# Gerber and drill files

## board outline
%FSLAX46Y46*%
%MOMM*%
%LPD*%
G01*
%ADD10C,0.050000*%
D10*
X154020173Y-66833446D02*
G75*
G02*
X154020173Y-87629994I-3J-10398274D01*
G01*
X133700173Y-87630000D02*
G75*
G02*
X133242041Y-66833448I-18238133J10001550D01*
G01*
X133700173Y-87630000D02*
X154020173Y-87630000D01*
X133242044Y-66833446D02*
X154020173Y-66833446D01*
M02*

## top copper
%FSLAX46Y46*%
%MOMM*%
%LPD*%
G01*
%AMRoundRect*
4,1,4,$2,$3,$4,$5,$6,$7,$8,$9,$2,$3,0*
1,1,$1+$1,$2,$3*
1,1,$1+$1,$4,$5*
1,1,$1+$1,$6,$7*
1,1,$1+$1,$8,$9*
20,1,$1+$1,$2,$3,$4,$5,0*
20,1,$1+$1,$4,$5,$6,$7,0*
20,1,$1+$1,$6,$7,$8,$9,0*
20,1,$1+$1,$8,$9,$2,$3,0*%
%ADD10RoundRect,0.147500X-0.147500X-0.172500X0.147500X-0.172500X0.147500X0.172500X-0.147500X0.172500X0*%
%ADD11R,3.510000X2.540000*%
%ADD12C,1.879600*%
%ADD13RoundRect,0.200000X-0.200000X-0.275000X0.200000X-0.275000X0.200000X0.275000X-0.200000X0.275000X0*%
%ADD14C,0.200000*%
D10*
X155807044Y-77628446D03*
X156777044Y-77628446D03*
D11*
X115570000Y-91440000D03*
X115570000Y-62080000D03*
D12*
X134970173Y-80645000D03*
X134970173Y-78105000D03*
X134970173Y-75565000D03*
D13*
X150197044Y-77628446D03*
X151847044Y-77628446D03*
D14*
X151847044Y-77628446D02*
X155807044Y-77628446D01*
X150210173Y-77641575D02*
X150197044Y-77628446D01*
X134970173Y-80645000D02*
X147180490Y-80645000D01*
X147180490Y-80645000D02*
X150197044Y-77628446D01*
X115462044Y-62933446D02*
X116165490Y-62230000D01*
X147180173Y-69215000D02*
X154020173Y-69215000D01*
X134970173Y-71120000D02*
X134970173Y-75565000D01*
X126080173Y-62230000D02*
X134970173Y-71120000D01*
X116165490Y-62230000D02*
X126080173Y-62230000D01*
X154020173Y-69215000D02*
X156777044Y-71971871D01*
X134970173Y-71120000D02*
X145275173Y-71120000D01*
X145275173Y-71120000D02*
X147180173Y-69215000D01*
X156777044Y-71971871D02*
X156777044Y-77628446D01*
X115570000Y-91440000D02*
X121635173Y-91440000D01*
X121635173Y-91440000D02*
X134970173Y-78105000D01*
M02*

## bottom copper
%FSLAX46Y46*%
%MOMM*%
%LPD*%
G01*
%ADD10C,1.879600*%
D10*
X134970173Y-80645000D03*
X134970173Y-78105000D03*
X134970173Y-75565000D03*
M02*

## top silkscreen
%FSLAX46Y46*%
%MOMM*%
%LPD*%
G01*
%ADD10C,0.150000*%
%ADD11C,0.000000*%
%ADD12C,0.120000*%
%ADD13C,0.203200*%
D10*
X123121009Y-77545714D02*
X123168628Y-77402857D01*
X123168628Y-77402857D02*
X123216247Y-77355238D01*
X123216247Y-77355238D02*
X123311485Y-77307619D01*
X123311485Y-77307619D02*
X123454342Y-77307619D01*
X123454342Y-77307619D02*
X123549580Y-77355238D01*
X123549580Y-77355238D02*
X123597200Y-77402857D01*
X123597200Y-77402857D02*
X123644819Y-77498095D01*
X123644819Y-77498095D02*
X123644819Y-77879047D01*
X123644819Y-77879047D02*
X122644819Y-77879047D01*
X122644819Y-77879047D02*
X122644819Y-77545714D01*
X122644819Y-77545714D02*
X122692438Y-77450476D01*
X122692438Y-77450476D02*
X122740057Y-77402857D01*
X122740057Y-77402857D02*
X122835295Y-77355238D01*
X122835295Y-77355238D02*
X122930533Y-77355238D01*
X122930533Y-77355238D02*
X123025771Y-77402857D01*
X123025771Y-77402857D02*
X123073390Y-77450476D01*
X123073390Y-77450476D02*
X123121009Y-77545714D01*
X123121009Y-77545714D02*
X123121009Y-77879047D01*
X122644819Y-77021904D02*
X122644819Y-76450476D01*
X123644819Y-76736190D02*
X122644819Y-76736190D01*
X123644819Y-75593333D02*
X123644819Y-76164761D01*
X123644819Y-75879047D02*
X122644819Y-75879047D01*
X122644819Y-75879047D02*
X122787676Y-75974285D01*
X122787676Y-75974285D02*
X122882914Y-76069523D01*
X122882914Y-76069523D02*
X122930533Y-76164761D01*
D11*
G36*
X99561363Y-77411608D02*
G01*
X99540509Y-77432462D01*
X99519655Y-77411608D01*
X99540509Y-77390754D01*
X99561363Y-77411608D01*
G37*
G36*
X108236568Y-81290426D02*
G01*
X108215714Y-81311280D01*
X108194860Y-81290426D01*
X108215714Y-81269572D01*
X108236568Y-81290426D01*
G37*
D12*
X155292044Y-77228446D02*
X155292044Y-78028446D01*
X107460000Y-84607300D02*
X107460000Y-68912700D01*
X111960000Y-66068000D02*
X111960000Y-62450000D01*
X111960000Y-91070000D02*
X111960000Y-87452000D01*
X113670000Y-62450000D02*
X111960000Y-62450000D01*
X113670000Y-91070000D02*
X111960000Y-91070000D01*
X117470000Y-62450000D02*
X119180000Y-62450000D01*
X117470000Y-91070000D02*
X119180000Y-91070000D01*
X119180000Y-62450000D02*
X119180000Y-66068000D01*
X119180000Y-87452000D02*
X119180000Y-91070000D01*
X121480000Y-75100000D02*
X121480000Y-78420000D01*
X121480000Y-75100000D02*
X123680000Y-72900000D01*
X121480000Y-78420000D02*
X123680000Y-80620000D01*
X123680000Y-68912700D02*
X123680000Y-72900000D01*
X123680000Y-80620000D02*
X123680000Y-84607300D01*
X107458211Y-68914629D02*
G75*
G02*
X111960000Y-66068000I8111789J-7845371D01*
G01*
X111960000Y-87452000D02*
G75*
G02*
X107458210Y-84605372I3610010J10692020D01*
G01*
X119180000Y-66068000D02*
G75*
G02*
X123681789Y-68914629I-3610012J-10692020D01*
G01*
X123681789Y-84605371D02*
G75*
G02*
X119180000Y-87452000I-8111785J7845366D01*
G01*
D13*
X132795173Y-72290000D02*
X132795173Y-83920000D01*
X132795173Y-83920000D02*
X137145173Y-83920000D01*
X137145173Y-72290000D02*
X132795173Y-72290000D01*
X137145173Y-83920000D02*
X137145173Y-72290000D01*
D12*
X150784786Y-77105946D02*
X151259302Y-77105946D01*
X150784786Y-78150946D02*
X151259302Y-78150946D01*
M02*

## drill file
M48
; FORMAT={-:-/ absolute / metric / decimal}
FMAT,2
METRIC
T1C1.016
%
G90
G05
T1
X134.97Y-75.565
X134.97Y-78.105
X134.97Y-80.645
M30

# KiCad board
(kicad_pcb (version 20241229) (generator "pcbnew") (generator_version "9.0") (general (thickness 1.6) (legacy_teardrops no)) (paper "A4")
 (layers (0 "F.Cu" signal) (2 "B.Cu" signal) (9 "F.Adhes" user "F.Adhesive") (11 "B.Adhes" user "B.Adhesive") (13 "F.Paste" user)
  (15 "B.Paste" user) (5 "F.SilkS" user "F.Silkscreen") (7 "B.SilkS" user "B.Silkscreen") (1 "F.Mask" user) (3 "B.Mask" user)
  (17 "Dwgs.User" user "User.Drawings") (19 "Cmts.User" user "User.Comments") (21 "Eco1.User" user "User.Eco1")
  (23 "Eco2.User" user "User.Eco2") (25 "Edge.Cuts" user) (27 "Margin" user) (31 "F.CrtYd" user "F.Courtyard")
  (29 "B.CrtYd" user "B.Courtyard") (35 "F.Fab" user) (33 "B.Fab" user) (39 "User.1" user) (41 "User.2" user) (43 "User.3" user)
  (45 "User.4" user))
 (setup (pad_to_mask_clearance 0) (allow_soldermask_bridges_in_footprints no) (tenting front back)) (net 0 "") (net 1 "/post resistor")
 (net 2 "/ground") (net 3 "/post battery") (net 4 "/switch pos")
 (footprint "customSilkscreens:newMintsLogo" (layer "F.Cu") (at 115.285173 74.93)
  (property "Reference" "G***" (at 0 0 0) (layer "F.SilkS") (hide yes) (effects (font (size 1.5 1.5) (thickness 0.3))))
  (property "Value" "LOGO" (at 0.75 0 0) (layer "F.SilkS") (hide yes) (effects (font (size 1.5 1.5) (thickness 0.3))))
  (fp_poly
   (pts (xy -15.72381 2.481608) (xy -15.744664 2.502462) (xy -15.765518 2.481608) (xy -15.744664 2.460754)) (stroke (width 0) (type solid))
   (fill yes) (layer "F.SilkS"))
  (fp_poly
   (pts (xy -7.048605 6.360426) (xy -7.069459 6.38128) (xy -7.090313 6.360426) (xy -7.069459 6.339572)) (stroke (width 0) (type solid))
   (fill yes) (layer "F.SilkS")))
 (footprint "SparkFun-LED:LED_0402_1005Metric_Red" (layer "F.Cu") (at 156.292044 77.628446)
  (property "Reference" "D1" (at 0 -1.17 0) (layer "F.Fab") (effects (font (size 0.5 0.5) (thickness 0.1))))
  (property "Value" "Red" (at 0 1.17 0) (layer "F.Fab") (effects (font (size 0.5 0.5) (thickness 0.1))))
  (fp_line (start -1 -0.4) (end -1 0.4) (stroke (width 0.12) (type solid)) (layer "F.SilkS"))
  (pad "1" smd roundrect (at -0.485 0) (size 0.59 0.64) (layers "F.Cu" "F.Mask" "F.Paste") (roundrect_rratio 0.25) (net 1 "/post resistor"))
  (pad "2" smd roundrect (at 0.485 0) (size 0.59 0.64) (layers "F.Cu" "F.Mask" "F.Paste") (roundrect_rratio 0.25) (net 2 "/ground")))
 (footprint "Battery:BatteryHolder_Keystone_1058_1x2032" (layer "F.Cu") (at 115.57 76.76 90)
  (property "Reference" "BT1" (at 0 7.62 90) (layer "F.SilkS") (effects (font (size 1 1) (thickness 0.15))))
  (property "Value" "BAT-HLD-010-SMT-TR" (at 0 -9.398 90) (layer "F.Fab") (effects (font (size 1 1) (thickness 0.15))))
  (fp_line (start -7.8473 -8.11) (end 7.8473 -8.11) (stroke (width 0.12) (type solid)) (layer "F.SilkS"))
  (fp_line (start 10.692 -3.61) (end 14.31 -3.61) (stroke (width 0.12) (type solid)) (layer "F.SilkS"))
  (fp_line (start -14.31 -3.61) (end -10.692 -3.61) (stroke (width 0.12) (type solid)) (layer "F.SilkS"))
  (fp_line (start 14.31 -1.9) (end 14.31 -3.61) (stroke (width 0.12) (type solid)) (layer "F.SilkS"))
  (fp_line (start -14.31 -1.9) (end -14.31 -3.61) (stroke (width 0.12) (type solid)) (layer "F.SilkS"))
  (fp_line (start 14.31 1.9) (end 14.31 3.61) (stroke (width 0.12) (type solid)) (layer "F.SilkS"))
  (fp_line (start -14.31 1.9) (end -14.31 3.61) (stroke (width 0.12) (type solid)) (layer "F.SilkS"))
  (fp_line (start 14.31 3.61) (end 10.692 3.61) (stroke (width 0.12) (type solid)) (layer "F.SilkS"))
  (fp_line (start -10.692 3.61) (end -14.31 3.61) (stroke (width 0.12) (type solid)) (layer "F.SilkS"))
  (fp_line (start 1.66 5.91) (end -1.66 5.91) (stroke (width 0.12) (type solid)) (layer "F.SilkS"))
  (fp_line (start 1.66 5.91) (end 3.86 8.11) (stroke (width 0.12) (type solid)) (layer "F.SilkS"))
  (fp_line (start -1.66 5.91) (end -3.86 8.11) (stroke (width 0.12) (type solid)) (layer "F.SilkS"))
  (fp_line (start 7.8473 8.11) (end 3.86 8.11) (stroke (width 0.12) (type solid)) (layer "F.SilkS"))
  (fp_line (start -3.86 8.11) (end -7.8473 8.11) (stroke (width 0.12) (type solid)) (layer "F.SilkS"))
  (fp_arc (start 7.845371 -8.111789) (mid 9.538085 -6.031244) (end 10.692 -3.61) (stroke (width 0.12) (type solid)) (layer "F.SilkS"))
  (fp_arc (start -10.692 -3.61) (mid -9.538084 -6.031244) (end -7.845371 -8.111789) (stroke (width 0.12) (type solid)) (layer "F.SilkS"))
  (fp_arc (start 10.692 3.61) (mid 9.538084 6.031244) (end 7.845371 8.111789) (stroke (width 0.12) (type solid)) (layer "F.SilkS"))
  (fp_arc (start -7.845371 8.111789) (mid -9.538085 6.031244) (end -10.692 3.61) (stroke (width 0.12) (type solid)) (layer "F.SilkS"))
  (pad "1" smd rect (at -14.68 0 90) (size 2.54 3.51) (layers "F.Cu" "F.Mask" "F.Paste") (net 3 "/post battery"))
  (pad "2" smd rect (at 14.68 0 90) (size 2.54 3.51) (layers "F.Cu" "F.Mask" "F.Paste") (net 2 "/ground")))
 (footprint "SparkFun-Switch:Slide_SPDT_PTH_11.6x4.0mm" (layer "F.Cu") (at 134.970173 78.105 180)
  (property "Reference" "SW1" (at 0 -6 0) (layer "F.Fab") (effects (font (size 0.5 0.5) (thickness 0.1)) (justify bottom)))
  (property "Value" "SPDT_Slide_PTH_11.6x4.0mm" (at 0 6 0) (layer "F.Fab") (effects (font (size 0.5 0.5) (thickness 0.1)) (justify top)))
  (fp_line (start 2.175 5.815) (end 2.175 -5.815) (stroke (width 0.2032) (type solid)) (layer "F.SilkS"))
  (fp_line (start 2.175 -5.815) (end -2.175 -5.815) (stroke (width 0.2032) (type solid)) (layer "F.SilkS"))
  (fp_line (start -2.175 5.815) (end 2.175 5.815) (stroke (width 0.2032) (type solid)) (layer "F.SilkS"))
  (fp_line (start -2.175 -5.815) (end -2.175 5.815) (stroke (width 0.2032) (type solid)) (layer "F.SilkS"))
  (pad "1" thru_hole circle (at 0 -2.54 180) (size 1.8796 1.8796) (drill 1.016) (layers "*.Cu" "*.Mask") (remove_unused_layers no)
   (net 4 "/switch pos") (thermal_bridge_angle 0))
  (pad "2" thru_hole circle (at 0 0 180) (size 1.8796 1.8796) (drill 1.016) (layers "*.Cu" "*.Mask") (remove_unused_layers no)
   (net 3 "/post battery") (thermal_bridge_angle 0))
  (pad "3" thru_hole circle (at 0 2.54 180) (size 1.8796 1.8796) (drill 1.016) (layers "*.Cu" "*.Mask") (remove_unused_layers no)
   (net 2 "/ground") (thermal_bridge_angle 0)))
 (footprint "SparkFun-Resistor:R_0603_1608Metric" (layer "F.Cu") (at 151.022044 77.628446)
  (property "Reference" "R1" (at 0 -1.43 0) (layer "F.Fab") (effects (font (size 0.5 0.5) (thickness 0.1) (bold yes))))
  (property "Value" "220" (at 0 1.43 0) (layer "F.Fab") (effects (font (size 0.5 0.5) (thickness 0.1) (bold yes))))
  (fp_line (start -0.237258 -0.5225) (end 0.237258 -0.5225) (stroke (width 0.12) (type solid)) (layer "F.SilkS"))
  (fp_line (start -0.237258 0.5225) (end 0.237258 0.5225) (stroke (width 0.12) (type solid)) (layer "F.SilkS"))
  (pad "1" smd roundrect (at -0.825 0) (size 0.8 0.95) (layers "F.Cu" "F.Mask" "F.Paste") (roundrect_rratio 0.25) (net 4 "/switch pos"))
  (pad "2" smd roundrect (at 0.825 0) (size 0.8 0.95) (layers "F.Cu" "F.Mask" "F.Paste") (roundrect_rratio 0.25) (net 1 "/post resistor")))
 (gr_arc (start 154.020173 66.833446) (mid 164.41845 77.231723) (end 154.020173 87.63) (stroke (width 0.05) (type default))
  (layer "Edge.Cuts"))
 (gr_arc (start 133.700173 87.63) (mid 94.666598 78.08655) (end 133.242044 66.833446) (stroke (width 0.05) (type default))
  (layer "Edge.Cuts"))
 (gr_line (start 133.700173 87.63) (end 154.020173 87.63) (stroke (width 0.05) (type default)) (layer "Edge.Cuts"))
 (gr_line (start 133.242044 66.833446) (end 154.020173 66.833446) (stroke (width 0.05) (type default)) (layer "Edge.Cuts"))
 (segment (start 151.847044 77.628446) (end 155.807044 77.628446) (width 0.2) (layer "F.Cu") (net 1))
 (segment (start 150.210173 77.641575) (end 150.197044 77.628446) (width 0.2) (layer "F.Cu") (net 4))
 (segment (start 134.970173 80.645) (end 147.18049 80.645) (width 0.2) (layer "F.Cu") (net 4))
 (segment (start 147.18049 80.645) (end 150.197044 77.628446) (width 0.2) (layer "F.Cu") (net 4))
 (segment (start 115.462044 62.933446) (end 116.16549 62.23) (width 0.2) (layer "F.Cu") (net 2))
 (segment (start 147.180173 69.215) (end 154.020173 69.215) (width 0.2) (layer "F.Cu") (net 2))
 (segment (start 134.970173 71.12) (end 134.970173 75.565) (width 0.2) (layer "F.Cu") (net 2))
 (segment (start 126.080173 62.23) (end 134.970173 71.12) (width 0.2) (layer "F.Cu") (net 2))
 (segment (start 116.16549 62.23) (end 126.080173 62.23) (width 0.2) (layer "F.Cu") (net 2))
 (segment (start 154.020173 69.215) (end 156.777044 71.971871) (width 0.2) (layer "F.Cu") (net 2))
 (segment (start 134.970173 71.12) (end 145.275173 71.12) (width 0.2) (layer "F.Cu") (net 2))
 (segment (start 145.275173 71.12) (end 147.180173 69.215) (width 0.2) (layer "F.Cu") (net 2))
 (segment (start 156.777044 71.971871) (end 156.777044 77.628446) (width 0.2) (layer "F.Cu") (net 2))
 (segment (start 115.57 91.44) (end 121.635173 91.44) (width 0.2) (layer "F.Cu") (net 3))
 (segment (start 121.635173 91.44) (end 134.970173 78.105) (width 0.2) (layer "F.Cu") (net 3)))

